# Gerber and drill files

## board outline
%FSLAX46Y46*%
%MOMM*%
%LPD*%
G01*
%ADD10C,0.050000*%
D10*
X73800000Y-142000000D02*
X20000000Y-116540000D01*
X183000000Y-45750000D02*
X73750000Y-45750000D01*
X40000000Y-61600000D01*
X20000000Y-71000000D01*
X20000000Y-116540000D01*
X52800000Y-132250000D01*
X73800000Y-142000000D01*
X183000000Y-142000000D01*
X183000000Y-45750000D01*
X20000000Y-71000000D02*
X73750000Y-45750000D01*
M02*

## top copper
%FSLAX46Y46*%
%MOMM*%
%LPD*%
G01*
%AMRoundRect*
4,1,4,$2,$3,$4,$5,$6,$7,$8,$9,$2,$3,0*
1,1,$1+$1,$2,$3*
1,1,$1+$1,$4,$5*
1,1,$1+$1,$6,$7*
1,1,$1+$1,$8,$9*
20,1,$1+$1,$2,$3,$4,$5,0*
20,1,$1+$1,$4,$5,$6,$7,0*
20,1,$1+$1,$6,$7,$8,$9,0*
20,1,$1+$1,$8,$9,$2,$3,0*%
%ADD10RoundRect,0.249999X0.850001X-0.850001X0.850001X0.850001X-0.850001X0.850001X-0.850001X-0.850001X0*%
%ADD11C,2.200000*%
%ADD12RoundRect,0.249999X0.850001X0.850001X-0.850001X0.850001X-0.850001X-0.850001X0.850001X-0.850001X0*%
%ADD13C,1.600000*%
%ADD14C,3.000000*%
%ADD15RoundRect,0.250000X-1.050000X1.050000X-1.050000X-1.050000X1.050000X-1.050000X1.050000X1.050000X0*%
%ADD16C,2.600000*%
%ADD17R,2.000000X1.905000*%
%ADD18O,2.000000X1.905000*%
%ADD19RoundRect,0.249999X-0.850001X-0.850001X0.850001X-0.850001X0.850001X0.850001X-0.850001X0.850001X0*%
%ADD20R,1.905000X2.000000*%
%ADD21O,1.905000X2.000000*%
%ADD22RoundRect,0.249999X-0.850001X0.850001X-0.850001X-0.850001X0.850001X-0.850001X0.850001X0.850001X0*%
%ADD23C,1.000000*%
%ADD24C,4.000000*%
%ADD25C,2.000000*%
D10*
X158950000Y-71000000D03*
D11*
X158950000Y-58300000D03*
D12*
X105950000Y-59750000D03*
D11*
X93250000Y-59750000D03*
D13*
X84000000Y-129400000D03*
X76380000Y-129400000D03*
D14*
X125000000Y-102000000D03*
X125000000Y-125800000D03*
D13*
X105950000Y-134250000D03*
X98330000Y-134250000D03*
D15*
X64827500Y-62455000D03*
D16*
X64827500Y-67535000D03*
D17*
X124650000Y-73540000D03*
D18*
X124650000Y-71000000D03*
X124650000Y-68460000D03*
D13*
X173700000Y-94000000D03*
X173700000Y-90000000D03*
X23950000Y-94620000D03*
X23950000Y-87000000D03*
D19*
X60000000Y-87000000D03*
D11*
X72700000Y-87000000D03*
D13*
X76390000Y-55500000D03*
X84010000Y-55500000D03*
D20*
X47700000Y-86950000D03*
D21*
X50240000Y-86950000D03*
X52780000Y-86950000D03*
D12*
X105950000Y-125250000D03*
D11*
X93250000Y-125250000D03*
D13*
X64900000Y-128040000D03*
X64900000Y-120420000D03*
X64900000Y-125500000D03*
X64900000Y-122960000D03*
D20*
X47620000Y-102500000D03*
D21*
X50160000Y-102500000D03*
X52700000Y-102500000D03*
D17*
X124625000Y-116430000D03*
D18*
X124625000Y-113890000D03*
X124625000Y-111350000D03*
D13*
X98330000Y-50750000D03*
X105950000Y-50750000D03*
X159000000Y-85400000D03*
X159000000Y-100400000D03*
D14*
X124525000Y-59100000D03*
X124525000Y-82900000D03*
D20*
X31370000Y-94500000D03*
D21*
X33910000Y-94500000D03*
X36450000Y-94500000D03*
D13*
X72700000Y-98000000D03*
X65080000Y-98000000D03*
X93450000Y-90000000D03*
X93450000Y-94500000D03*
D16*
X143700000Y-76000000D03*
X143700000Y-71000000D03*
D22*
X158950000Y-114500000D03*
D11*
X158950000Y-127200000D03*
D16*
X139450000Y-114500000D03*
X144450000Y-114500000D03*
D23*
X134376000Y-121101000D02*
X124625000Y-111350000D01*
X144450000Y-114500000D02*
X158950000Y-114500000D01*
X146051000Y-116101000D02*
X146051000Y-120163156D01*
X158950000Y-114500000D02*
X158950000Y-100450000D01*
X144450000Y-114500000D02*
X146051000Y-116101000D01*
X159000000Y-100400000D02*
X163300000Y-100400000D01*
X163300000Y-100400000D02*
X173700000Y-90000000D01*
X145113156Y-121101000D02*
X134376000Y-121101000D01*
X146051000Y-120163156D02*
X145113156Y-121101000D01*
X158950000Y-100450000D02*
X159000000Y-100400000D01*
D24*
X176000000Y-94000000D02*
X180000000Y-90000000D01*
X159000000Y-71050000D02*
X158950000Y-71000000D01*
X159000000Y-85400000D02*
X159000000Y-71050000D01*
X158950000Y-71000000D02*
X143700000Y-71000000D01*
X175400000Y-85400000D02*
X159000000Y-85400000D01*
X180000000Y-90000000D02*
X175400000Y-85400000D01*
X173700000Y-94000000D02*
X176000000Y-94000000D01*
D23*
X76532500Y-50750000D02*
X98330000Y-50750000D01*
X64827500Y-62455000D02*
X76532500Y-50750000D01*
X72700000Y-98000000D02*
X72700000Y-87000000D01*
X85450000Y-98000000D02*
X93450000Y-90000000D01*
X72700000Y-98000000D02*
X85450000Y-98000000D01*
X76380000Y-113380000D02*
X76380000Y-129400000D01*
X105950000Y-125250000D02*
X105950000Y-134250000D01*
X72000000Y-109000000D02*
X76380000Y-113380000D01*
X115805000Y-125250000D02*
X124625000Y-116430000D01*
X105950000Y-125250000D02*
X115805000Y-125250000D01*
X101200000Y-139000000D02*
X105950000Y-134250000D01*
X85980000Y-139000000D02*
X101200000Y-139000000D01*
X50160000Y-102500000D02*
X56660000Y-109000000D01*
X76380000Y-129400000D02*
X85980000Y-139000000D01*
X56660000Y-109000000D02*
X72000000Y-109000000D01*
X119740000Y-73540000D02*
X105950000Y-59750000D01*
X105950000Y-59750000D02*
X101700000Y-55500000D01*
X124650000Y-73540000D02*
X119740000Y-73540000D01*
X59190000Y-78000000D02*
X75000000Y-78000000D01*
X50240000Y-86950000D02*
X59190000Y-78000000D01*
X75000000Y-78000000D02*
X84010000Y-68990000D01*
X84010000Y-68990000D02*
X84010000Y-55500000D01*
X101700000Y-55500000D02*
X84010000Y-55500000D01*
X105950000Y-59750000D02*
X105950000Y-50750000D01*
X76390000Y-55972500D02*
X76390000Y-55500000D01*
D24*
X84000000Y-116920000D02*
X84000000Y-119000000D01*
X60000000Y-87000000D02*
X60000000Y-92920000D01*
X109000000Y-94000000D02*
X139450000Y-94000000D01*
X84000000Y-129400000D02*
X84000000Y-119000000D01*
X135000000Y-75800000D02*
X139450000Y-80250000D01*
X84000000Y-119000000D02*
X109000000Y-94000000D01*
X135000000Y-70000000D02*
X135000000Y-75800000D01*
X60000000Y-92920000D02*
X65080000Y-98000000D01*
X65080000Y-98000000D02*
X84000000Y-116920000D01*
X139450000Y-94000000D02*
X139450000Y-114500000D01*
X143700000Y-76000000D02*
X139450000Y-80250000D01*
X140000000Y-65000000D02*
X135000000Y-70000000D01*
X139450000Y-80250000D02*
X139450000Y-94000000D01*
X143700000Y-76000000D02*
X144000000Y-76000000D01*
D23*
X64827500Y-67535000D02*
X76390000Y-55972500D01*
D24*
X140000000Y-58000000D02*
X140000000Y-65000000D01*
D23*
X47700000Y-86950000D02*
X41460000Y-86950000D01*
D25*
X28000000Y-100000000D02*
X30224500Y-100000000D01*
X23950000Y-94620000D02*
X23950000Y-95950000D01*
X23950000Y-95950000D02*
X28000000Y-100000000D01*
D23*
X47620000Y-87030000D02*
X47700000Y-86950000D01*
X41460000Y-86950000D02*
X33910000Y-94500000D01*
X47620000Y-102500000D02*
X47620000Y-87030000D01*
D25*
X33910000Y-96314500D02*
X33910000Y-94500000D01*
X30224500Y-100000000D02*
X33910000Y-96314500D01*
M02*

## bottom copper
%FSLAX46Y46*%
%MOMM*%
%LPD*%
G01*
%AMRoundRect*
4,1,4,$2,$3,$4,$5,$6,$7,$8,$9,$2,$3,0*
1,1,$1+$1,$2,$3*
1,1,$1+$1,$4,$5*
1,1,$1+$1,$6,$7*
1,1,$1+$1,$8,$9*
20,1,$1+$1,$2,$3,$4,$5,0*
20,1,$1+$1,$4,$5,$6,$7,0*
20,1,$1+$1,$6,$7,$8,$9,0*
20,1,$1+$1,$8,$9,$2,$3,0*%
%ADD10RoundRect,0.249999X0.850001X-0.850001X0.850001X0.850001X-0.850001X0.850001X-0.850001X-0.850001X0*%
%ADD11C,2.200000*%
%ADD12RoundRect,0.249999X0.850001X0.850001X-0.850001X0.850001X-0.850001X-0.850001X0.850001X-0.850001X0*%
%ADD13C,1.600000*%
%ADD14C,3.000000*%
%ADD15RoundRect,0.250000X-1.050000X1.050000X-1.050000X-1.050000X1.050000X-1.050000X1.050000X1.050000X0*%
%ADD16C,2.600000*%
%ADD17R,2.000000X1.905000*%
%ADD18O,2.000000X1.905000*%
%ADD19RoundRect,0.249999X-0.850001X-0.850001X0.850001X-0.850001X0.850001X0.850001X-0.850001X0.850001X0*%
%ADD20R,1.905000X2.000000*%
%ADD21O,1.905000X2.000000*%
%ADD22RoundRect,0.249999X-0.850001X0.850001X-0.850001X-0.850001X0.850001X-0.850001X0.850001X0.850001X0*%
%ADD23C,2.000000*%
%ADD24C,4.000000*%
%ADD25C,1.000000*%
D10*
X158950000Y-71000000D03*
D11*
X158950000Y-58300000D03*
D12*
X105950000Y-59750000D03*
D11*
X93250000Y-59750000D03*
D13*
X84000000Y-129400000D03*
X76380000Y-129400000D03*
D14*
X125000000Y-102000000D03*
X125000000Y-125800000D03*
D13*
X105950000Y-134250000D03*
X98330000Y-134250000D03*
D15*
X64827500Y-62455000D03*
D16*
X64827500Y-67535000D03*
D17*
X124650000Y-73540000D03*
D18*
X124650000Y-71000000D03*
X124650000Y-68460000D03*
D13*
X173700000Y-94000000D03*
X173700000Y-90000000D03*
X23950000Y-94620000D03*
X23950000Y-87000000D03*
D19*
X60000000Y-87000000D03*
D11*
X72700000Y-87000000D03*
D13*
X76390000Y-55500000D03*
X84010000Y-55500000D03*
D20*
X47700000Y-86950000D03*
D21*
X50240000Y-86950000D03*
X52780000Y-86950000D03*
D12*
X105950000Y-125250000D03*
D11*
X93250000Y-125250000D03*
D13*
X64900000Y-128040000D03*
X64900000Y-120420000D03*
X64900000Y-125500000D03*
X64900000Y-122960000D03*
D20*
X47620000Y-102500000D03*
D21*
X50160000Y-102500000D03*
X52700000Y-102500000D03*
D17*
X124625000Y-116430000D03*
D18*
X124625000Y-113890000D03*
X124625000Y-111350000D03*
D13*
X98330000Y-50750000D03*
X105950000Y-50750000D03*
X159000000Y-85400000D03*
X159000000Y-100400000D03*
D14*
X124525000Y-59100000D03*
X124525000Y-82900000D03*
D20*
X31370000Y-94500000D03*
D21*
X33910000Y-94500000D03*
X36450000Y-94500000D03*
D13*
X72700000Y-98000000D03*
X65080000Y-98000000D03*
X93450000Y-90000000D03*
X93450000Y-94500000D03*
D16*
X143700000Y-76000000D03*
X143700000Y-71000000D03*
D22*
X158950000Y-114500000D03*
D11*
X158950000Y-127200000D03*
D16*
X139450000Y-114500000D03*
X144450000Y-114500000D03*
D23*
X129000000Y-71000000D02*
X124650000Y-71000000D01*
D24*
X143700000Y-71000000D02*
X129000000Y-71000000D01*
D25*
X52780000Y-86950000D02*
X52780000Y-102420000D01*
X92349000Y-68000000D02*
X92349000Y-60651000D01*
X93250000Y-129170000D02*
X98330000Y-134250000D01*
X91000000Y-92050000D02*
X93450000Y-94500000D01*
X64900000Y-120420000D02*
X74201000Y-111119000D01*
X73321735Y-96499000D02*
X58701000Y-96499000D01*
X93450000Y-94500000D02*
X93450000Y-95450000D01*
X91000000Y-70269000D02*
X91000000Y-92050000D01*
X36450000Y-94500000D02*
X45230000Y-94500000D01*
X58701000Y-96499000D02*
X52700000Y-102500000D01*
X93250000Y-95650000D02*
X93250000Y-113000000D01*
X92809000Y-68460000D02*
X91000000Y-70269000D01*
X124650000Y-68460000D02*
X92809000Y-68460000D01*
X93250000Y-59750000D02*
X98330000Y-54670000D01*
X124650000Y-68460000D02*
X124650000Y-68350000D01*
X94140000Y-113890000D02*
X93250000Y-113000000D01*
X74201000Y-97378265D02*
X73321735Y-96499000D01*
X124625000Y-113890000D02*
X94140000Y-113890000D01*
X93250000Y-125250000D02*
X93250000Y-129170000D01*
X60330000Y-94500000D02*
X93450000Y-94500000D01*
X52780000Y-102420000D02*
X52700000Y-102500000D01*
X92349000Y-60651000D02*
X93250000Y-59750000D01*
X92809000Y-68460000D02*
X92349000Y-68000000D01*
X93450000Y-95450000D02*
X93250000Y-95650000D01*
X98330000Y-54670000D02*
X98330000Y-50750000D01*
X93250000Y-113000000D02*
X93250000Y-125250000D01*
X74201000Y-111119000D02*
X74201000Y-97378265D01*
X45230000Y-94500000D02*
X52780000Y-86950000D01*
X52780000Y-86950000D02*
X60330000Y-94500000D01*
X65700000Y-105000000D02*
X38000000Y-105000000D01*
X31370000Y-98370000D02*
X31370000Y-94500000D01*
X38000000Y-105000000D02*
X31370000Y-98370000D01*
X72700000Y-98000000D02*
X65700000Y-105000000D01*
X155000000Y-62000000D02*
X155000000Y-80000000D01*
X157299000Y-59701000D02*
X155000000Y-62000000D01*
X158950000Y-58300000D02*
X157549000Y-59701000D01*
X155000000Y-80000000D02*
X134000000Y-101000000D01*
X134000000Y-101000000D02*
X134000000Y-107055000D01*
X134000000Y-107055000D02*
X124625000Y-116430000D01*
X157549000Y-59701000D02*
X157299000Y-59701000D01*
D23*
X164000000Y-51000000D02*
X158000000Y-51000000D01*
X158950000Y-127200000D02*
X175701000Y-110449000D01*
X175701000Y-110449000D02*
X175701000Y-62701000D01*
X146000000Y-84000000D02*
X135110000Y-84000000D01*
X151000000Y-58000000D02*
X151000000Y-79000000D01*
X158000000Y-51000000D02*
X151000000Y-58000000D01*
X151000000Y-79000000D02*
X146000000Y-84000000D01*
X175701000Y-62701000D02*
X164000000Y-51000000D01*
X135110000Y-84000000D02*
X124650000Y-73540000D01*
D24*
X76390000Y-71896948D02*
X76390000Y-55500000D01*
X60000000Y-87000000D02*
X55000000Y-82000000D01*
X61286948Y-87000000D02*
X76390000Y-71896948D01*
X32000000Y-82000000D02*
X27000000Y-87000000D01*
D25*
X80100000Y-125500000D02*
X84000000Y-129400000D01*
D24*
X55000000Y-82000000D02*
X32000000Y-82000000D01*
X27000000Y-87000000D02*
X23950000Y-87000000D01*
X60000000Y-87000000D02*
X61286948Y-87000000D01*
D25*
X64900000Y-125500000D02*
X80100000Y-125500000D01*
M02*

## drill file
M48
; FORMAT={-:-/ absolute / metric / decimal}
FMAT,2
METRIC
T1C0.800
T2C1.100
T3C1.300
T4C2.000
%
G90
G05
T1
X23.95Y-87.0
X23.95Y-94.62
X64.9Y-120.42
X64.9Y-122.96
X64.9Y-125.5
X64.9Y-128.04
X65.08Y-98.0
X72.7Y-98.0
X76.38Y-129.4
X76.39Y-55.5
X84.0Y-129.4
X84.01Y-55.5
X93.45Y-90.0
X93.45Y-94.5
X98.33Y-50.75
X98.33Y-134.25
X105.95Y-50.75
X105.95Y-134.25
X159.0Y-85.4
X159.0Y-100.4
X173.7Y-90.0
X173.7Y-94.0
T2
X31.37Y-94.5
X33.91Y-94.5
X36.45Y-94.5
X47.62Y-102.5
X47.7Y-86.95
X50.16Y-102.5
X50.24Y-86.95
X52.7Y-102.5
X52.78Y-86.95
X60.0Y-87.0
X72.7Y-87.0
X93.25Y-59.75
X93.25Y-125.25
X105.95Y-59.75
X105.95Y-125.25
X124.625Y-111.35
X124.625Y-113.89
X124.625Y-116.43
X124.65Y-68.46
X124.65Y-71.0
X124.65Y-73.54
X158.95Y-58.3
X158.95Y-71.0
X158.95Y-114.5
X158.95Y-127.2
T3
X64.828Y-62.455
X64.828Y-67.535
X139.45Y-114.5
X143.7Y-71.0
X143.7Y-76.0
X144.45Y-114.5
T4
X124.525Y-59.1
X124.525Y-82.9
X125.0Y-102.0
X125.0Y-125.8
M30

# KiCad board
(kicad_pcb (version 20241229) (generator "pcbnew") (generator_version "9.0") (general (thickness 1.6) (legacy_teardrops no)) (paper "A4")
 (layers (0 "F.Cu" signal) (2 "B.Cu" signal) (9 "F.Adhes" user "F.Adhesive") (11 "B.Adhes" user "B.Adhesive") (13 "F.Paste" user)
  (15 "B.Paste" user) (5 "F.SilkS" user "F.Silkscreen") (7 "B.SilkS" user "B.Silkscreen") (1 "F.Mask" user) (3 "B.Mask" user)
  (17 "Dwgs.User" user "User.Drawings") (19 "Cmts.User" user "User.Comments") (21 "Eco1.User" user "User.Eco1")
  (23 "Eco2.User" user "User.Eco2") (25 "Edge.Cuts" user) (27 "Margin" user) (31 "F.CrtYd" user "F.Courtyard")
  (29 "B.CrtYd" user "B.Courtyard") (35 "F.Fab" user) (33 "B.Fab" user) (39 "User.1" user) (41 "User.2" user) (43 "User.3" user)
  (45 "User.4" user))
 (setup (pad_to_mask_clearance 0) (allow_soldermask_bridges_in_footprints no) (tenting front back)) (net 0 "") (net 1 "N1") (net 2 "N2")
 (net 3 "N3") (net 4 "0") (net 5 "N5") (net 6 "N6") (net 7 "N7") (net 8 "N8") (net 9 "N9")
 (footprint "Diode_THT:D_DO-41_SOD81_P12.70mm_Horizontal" (layer "F.Cu") (at 158.95 71 90)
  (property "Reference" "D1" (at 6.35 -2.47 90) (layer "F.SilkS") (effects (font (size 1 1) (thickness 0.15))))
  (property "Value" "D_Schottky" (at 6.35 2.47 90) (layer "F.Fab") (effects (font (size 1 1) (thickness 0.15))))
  (pad "1" thru_hole roundrect (at 0 0 90) (size 2.2 2.2) (drill 1.1) (layers "*.Cu" "*.Mask") (remove_unused_layers no)
   (roundrect_rratio 0.113636) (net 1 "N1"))
  (pad "2" thru_hole circle (at 12.7 0 90) (size 2.2 2.2) (drill 1.1) (layers "*.Cu" "*.Mask") (remove_unused_layers no) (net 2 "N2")))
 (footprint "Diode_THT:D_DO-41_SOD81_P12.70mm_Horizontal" (layer "F.Cu") (at 105.95 59.75 180)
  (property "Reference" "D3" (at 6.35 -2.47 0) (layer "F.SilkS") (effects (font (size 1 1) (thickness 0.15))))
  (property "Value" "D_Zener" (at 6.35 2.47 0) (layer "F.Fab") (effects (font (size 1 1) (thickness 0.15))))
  (pad "1" thru_hole roundrect (at 0 0 180) (size 2.2 2.2) (drill 1.1) (layers "*.Cu" "*.Mask") (remove_unused_layers no)
   (roundrect_rratio 0.113636) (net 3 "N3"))
  (pad "2" thru_hole circle (at 12.7 0 180) (size 2.2 2.2) (drill 1.1) (layers "*.Cu" "*.Mask") (remove_unused_layers no) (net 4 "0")))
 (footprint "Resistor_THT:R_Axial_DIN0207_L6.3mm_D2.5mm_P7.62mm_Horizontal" (layer "F.Cu") (at 84 129.4 180)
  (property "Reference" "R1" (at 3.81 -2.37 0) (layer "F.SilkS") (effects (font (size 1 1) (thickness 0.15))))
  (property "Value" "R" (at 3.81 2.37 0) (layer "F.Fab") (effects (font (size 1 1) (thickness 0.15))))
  (pad "1" thru_hole circle (at 0 0 180) (size 1.6 1.6) (drill 0.8) (layers "*.Cu" "*.Mask") (remove_unused_layers no) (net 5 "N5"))
  (pad "2" thru_hole circle (at 7.62 0 180) (size 1.6 1.6) (drill 0.8) (layers "*.Cu" "*.Mask") (remove_unused_layers no) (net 2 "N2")))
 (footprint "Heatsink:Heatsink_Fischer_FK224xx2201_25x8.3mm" (layer "F.Cu") (at 125 102 -90)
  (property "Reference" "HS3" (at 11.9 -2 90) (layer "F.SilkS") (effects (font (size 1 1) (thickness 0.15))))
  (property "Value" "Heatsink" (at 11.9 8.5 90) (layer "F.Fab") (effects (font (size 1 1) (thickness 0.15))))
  (pad "1" thru_hole circle (at 0 0 270) (size 3 3) (drill 2) (layers "*.Cu" "*.Mask") (remove_unused_layers no))
  (pad "1" thru_hole circle (at 23.8 0 270) (size 3 3) (drill 2) (layers "*.Cu" "*.Mask") (remove_unused_layers no)))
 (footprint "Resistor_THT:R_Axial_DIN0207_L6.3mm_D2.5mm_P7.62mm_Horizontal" (layer "F.Cu") (at 105.95 134.25 180)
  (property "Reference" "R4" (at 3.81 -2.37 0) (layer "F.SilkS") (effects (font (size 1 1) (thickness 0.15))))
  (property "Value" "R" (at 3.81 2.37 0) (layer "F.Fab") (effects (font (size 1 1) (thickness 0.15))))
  (pad "1" thru_hole circle (at 0 0 180) (size 1.6 1.6) (drill 0.8) (layers "*.Cu" "*.Mask") (remove_unused_layers no) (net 2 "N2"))
  (pad "2" thru_hole circle (at 7.62 0 180) (size 1.6 1.6) (drill 0.8) (layers "*.Cu" "*.Mask") (remove_unused_layers no) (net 4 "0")))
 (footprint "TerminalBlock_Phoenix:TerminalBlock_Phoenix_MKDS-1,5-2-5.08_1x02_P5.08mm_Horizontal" (layer "F.Cu") (at 64.8275 62.455 -90)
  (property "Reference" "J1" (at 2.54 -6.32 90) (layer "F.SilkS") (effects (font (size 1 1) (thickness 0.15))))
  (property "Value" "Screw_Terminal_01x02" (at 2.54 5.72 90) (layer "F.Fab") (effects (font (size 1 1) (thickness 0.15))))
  (pad "1" thru_hole roundrect (at 0 0 270) (size 2.6 2.6) (drill 1.3) (layers "*.Cu" "*.Mask") (remove_unused_layers no)
   (roundrect_rratio 0.096154) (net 4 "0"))
  (pad "2" thru_hole circle (at 5.08 0 270) (size 2.6 2.6) (drill 1.3) (layers "*.Cu" "*.Mask") (remove_unused_layers no) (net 5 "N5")))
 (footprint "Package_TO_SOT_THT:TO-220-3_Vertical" (layer "F.Cu") (at 124.65 73.54 90)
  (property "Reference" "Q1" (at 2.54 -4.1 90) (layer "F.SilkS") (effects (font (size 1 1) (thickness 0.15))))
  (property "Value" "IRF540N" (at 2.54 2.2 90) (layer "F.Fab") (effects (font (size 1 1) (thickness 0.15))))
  (pad "1" thru_hole rect (at 0 0 90) (size 1.905 2) (drill 1.1) (layers "*.Cu" "*.Mask") (remove_unused_layers no) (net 3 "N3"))
  (pad "2" thru_hole oval (at 2.54 0 90) (size 1.905 2) (drill 1.1) (layers "*.Cu" "*.Mask") (remove_unused_layers no) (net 1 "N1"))
  (pad "3" thru_hole oval (at 5.08 0 90) (size 1.905 2) (drill 1.1) (layers "*.Cu" "*.Mask") (remove_unused_layers no) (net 4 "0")))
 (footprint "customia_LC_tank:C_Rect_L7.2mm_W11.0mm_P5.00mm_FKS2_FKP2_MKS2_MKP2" (layer "F.Cu") (at 248.7 94.5 180)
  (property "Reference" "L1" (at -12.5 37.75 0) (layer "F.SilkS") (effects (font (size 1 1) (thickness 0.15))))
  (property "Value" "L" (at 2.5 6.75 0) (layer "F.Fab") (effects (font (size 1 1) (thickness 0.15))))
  (pad "1" thru_hole circle (at 75 0.5 180) (size 1.6 1.6) (drill 0.8) (layers "*.Cu" "*.Mask") (remove_unused_layers no) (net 1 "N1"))
  (pad "2" thru_hole circle (at 75 4.5 180) (size 1.6 1.6) (drill 0.8) (layers "*.Cu" "*.Mask") (remove_unused_layers no) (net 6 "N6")))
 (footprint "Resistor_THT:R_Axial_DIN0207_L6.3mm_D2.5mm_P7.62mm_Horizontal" (layer "F.Cu") (at 23.95 94.62 90)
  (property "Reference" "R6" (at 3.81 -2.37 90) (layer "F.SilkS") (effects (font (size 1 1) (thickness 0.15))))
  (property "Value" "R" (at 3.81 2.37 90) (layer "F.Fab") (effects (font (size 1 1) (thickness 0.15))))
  (pad "1" thru_hole circle (at 0 0 90) (size 1.6 1.6) (drill 0.8) (layers "*.Cu" "*.Mask") (remove_unused_layers no) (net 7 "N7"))
  (pad "2" thru_hole circle (at 7.62 0 90) (size 1.6 1.6) (drill 0.8) (layers "*.Cu" "*.Mask") (remove_unused_layers no) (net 5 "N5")))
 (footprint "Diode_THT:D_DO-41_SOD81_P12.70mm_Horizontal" (layer "F.Cu") (at 60 87)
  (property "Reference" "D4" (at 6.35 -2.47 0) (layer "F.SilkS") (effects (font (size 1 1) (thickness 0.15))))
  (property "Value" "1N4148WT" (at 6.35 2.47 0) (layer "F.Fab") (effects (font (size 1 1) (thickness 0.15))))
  (pad "1" thru_hole roundrect (at 0 0) (size 2.2 2.2) (drill 1.1) (layers "*.Cu" "*.Mask") (remove_unused_layers no)
   (roundrect_rratio 0.113636) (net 5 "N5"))
  (pad "2" thru_hole circle (at 12.7 0) (size 2.2 2.2) (drill 1.1) (layers "*.Cu" "*.Mask") (remove_unused_layers no) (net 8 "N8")))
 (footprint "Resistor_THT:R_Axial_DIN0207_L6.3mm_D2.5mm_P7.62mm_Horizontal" (layer "F.Cu") (at 76.39 55.5)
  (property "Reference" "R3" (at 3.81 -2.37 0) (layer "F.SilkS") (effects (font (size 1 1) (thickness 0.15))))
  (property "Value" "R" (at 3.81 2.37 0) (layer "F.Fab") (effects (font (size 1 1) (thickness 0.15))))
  (pad "1" thru_hole circle (at 0 0) (size 1.6 1.6) (drill 0.8) (layers "*.Cu" "*.Mask") (remove_unused_layers no) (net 5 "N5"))
  (pad "2" thru_hole circle (at 7.62 0) (size 1.6 1.6) (drill 0.8) (layers "*.Cu" "*.Mask") (remove_unused_layers no) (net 3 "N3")))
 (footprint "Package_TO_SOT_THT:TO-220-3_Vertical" (layer "F.Cu") (at 47.7 86.95)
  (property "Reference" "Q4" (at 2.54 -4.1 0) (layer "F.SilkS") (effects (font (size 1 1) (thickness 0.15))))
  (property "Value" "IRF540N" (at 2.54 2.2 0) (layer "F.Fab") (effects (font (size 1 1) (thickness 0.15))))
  (pad "1" thru_hole rect (at 0 0) (size 1.905 2) (drill 1.1) (layers "*.Cu" "*.Mask") (remove_unused_layers no) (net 7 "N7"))
  (pad "2" thru_hole oval (at 2.54 0) (size 1.905 2) (drill 1.1) (layers "*.Cu" "*.Mask") (remove_unused_layers no) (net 3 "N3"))
  (pad "3" thru_hole oval (at 5.08 0) (size 1.905 2) (drill 1.1) (layers "*.Cu" "*.Mask") (remove_unused_layers no) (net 4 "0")))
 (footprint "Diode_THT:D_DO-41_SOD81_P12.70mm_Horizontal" (layer "F.Cu") (at 105.95 125.25 180)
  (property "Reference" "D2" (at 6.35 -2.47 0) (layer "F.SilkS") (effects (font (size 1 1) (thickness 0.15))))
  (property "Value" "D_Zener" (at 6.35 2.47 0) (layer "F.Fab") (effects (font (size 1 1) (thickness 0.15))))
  (pad "1" thru_hole roundrect (at 0 0 180) (size 2.2 2.2) (drill 1.1) (layers "*.Cu" "*.Mask") (remove_unused_layers no)
   (roundrect_rratio 0.113636) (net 2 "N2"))
  (pad "2" thru_hole circle (at 12.7 0 180) (size 2.2 2.2) (drill 1.1) (layers "*.Cu" "*.Mask") (remove_unused_layers no) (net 4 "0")))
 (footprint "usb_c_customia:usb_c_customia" (layer "F.Cu") (at 64.9 128.04 90)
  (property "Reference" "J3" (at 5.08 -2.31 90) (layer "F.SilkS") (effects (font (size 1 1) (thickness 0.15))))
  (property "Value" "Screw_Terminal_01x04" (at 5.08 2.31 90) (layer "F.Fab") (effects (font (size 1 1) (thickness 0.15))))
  (pad "2" thru_hole circle (at 0 0 90) (size 1.6 1.6) (drill 0.8) (layers "*.Cu" "*.Mask") (remove_unused_layers no) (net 4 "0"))
  (pad "2" thru_hole circle (at 7.62 0 90) (size 1.6 1.6) (drill 0.8) (layers "*.Cu" "*.Mask") (remove_unused_layers no) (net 4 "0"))
  (pad "3" thru_hole circle (at 2.54 0 90) (size 1.6 1.6) (drill 0.8) (layers "*.Cu" "*.Mask") (remove_unused_layers no) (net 5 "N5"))
  (pad "4" thru_hole circle (at 5.08 0 90) (size 1.6 1.6) (drill 0.8) (layers "*.Cu" "*.Mask") (remove_unused_layers no) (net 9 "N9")))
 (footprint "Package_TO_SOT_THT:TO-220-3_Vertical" (layer "F.Cu") (at 47.62 102.5)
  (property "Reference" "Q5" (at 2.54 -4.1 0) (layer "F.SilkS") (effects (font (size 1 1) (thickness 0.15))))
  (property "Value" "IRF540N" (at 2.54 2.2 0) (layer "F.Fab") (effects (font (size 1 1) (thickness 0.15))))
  (pad "1" thru_hole rect (at 0 0) (size 1.905 2) (drill 1.1) (layers "*.Cu" "*.Mask") (remove_unused_layers no) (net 7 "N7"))
  (pad "2" thru_hole oval (at 2.54 0) (size 1.905 2) (drill 1.1) (layers "*.Cu" "*.Mask") (remove_unused_layers no) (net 2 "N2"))
  (pad "3" thru_hole oval (at 5.08 0) (size 1.905 2) (drill 1.1) (layers "*.Cu" "*.Mask") (remove_unused_layers no) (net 4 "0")))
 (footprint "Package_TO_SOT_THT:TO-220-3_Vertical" (layer "F.Cu") (at 124.625 116.43 90)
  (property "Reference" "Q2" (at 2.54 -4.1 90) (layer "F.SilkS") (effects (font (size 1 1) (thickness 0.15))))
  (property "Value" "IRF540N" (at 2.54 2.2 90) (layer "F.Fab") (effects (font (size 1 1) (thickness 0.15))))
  (pad "1" thru_hole rect (at 0 0 90) (size 1.905 2) (drill 1.1) (layers "*.Cu" "*.Mask") (remove_unused_layers no) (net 2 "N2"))
  (pad "2" thru_hole oval (at 2.54 0 90) (size 1.905 2) (drill 1.1) (layers "*.Cu" "*.Mask") (remove_unused_layers no) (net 4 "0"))
  (pad "3" thru_hole oval (at 5.08 0 90) (size 1.905 2) (drill 1.1) (layers "*.Cu" "*.Mask") (remove_unused_layers no) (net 6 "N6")))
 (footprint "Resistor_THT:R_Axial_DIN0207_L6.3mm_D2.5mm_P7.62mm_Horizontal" (layer "F.Cu") (at 98.33 50.75)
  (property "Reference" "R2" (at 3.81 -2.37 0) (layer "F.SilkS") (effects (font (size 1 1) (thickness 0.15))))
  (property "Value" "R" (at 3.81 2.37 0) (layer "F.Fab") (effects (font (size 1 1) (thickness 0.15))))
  (pad "1" thru_hole circle (at 0 0) (size 1.6 1.6) (drill 0.8) (layers "*.Cu" "*.Mask") (remove_unused_layers no) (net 4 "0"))
  (pad "2" thru_hole circle (at 7.62 0) (size 1.6 1.6) (drill 0.8) (layers "*.Cu" "*.Mask") (remove_unused_layers no) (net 3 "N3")))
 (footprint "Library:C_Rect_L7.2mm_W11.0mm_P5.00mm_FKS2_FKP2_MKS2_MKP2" (layer "F.Cu") (at 159.1 93.1 -90)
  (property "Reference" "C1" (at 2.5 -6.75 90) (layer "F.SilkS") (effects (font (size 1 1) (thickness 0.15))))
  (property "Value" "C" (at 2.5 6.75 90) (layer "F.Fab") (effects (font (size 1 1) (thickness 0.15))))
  (pad "1" thru_hole circle (at -7.7 0.1 270) (size 1.6 1.6) (drill 0.8) (layers "*.Cu" "*.Mask") (remove_unused_layers no) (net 1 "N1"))
  (pad "2" thru_hole circle (at 7.3 0.1 270) (size 1.6 1.6) (drill 0.8) (layers "*.Cu" "*.Mask") (remove_unused_layers no) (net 6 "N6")))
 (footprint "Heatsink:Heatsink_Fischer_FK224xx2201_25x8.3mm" (layer "F.Cu") (at 124.525 59.1 -90)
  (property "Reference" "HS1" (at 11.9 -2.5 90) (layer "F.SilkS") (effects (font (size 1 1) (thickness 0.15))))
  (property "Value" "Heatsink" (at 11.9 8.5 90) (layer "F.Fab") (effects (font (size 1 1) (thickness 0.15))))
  (pad "1" thru_hole circle (at 0 0 270) (size 3 3) (drill 2) (layers "*.Cu" "*.Mask") (remove_unused_layers no))
  (pad "1" thru_hole circle (at 23.8 0 270) (size 3 3) (drill 2) (layers "*.Cu" "*.Mask") (remove_unused_layers no)))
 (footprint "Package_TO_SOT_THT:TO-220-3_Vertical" (layer "F.Cu") (at 31.37 94.5)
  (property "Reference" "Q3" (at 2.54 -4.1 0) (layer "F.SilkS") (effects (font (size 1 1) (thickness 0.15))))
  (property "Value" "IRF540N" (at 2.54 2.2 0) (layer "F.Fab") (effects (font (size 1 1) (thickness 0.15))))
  (pad "1" thru_hole rect (at 0 0) (size 1.905 2) (drill 1.1) (layers "*.Cu" "*.Mask") (remove_unused_layers no) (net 8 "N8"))
  (pad "2" thru_hole oval (at 2.54 0) (size 1.905 2) (drill 1.1) (layers "*.Cu" "*.Mask") (remove_unused_layers no) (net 7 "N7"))
  (pad "3" thru_hole oval (at 5.08 0) (size 1.905 2) (drill 1.1) (layers "*.Cu" "*.Mask") (remove_unused_layers no) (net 4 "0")))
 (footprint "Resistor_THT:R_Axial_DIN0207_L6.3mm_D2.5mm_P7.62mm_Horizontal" (layer "F.Cu") (at 72.7 98 180)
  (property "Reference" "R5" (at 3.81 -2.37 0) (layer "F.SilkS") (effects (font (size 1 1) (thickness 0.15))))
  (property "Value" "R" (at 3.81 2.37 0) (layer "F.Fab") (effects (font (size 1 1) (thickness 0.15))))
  (pad "1" thru_hole circle (at 0 0 180) (size 1.6 1.6) (drill 0.8) (layers "*.Cu" "*.Mask") (remove_unused_layers no) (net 8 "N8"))
  (pad "2" thru_hole circle (at 7.62 0 180) (size 1.6 1.6) (drill 0.8) (layers "*.Cu" "*.Mask") (remove_unused_layers no) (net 5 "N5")))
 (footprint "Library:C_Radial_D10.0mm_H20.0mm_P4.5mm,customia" (layer "F.Cu") (at 93.45 89.75 -90)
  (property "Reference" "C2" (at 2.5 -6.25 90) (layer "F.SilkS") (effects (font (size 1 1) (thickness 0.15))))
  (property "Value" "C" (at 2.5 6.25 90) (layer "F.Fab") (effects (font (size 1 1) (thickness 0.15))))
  (pad "1" thru_hole circle (at 0.25 0 270) (size 1.6 1.6) (drill 0.8) (layers "*.Cu" "*.Mask") (remove_unused_layers no) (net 8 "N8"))
  (pad "2" thru_hole circle (at 4.75 0 270) (size 1.6 1.6) (drill 0.8) (layers "*.Cu" "*.Mask") (remove_unused_layers no) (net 4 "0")))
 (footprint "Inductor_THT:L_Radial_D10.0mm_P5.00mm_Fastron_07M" (layer "F.Cu") (at 143.7 76 90)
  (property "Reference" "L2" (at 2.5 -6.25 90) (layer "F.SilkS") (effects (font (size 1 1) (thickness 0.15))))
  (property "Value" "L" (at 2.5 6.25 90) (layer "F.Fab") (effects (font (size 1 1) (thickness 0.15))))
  (pad "1" thru_hole circle (at 0 0 90) (size 2.6 2.6) (drill 1.3) (layers "*.Cu" "*.Mask") (remove_unused_layers no) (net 5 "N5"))
  (pad "2" thru_hole circle (at 5 0 90) (size 2.6 2.6) (drill 1.3) (layers "*.Cu" "*.Mask") (remove_unused_layers no) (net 1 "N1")))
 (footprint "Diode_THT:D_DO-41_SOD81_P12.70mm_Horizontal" (layer "F.Cu") (at 158.95 114.5 -90)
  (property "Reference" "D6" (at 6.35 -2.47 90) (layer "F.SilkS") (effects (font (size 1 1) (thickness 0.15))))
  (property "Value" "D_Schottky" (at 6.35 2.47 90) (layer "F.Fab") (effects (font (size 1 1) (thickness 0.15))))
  (pad "1" thru_hole roundrect (at 0 0 270) (size 2.2 2.2) (drill 1.1) (layers "*.Cu" "*.Mask") (remove_unused_layers no)
   (roundrect_rratio 0.113636) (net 6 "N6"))
  (pad "2" thru_hole circle (at 12.7 0 270) (size 2.2 2.2) (drill 1.1) (layers "*.Cu" "*.Mask") (remove_unused_layers no) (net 3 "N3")))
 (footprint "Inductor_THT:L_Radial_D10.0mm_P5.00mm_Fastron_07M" (layer "F.Cu") (at 139.45 114.5)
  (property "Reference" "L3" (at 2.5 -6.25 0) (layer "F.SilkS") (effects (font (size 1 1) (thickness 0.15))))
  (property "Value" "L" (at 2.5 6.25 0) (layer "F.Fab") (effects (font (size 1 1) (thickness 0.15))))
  (pad "1" thru_hole circle (at 0 0) (size 2.6 2.6) (drill 1.3) (layers "*.Cu" "*.Mask") (remove_unused_layers no) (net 5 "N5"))
  (pad "2" thru_hole circle (at 5 0) (size 2.6 2.6) (drill 1.3) (layers "*.Cu" "*.Mask") (remove_unused_layers no) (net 6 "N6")))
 (gr_line (start 73.8 142) (end 20 116.54) (stroke (width 0.05) (type default)) (layer "Edge.Cuts"))
 (gr_poly
  (pts (xy 183 45.75) (xy 73.75 45.75) (xy 40 61.6) (xy 20 71) (xy 20 116.54) (xy 52.8 132.25) (xy 73.8 142) (xy 183 142))
  (stroke (width 0.05) (type solid)) (fill no) (layer "Edge.Cuts"))
 (gr_line (start 20 71) (end 73.75 45.75) (stroke (width 0.05) (type default)) (layer "Edge.Cuts"))
 (segment (start 134.376 121.101) (end 124.625 111.35) (width 1) (layer "F.Cu") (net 6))
 (segment (start 144.45 114.5) (end 158.95 114.5) (width 1) (layer "F.Cu") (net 6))
 (segment (start 146.051 116.101) (end 146.051 120.163156) (width 1) (layer "F.Cu") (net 6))
 (segment (start 158.95 114.5) (end 158.95 100.45) (width 1) (layer "F.Cu") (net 6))
 (segment (start 144.45 114.5) (end 146.051 116.101) (width 1) (layer "F.Cu") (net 6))
 (segment (start 159 100.4) (end 163.3 100.4) (width 1) (layer "F.Cu") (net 6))
 (segment (start 163.3 100.4) (end 173.7 90) (width 1) (layer "F.Cu") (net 6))
 (segment (start 145.113156 121.101) (end 134.376 121.101) (width 1) (layer "F.Cu") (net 6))
 (segment (start 146.051 120.163156) (end 145.113156 121.101) (width 1) (layer "F.Cu") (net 6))
 (segment (start 158.95 100.45) (end 159 100.4) (width 1) (layer "F.Cu") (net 6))
 (segment (start 176 94) (end 180 90) (width 4) (layer "F.Cu") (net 1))
 (segment (start 159 71.05) (end 158.95 71) (width 4) (layer "F.Cu") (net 1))
 (segment (start 159 85.4) (end 159 71.05) (width 4) (layer "F.Cu") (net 1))
 (segment (start 158.95 71) (end 143.7 71) (width 4) (layer "F.Cu") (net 1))
 (segment (start 175.4 85.4) (end 159 85.4) (width 4) (layer "F.Cu") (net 1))
 (segment (start 180 90) (end 175.4 85.4) (width 4) (layer "F.Cu") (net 1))
 (segment (start 173.7 94) (end 176 94) (width 4) (layer "F.Cu") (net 1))
 (segment (start 129 71) (end 124.65 71) (width 2) (layer "B.Cu") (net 1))
 (segment (start 143.7 71) (end 129 71) (width 4) (layer "B.Cu") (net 1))
 (segment (start 76.5325 50.75) (end 98.33 50.75) (width 1) (layer "F.Cu") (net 4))
 (segment (start 64.8275 62.455) (end 76.5325 50.75) (width 1) (layer "F.Cu") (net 4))
 (segment (start 52.78 86.95) (end 52.78 102.42) (width 1) (layer "B.Cu") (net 4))
 (segment (start 92.349 68) (end 92.349 60.651) (width 1) (layer "B.Cu") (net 4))
 (segment (start 93.25 129.17) (end 98.33 134.25) (width 1) (layer "B.Cu") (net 4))
 (segment (start 91 92.05) (end 93.45 94.5) (width 1) (layer "B.Cu") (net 4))
 (segment (start 64.9 120.42) (end 74.201 111.119) (width 1) (layer "B.Cu") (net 4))
 (segment (start 73.321735 96.499) (end 58.701 96.499) (width 1) (layer "B.Cu") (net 4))
 (segment (start 93.45 94.5) (end 93.45 95.45) (width 1) (layer "B.Cu") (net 4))
 (segment (start 91 70.269) (end 91 92.05) (width 1) (layer "B.Cu") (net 4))
 (segment (start 36.45 94.5) (end 45.23 94.5) (width 1) (layer "B.Cu") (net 4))
 (segment (start 58.701 96.499) (end 52.7 102.5) (width 1) (layer "B.Cu") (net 4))
 (segment (start 93.25 95.65) (end 93.25 113) (width 1) (layer "B.Cu") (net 4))
 (segment (start 92.809 68.46) (end 91 70.269) (width 1) (layer "B.Cu") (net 4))
 (segment (start 124.65 68.46) (end 92.809 68.46) (width 1) (layer "B.Cu") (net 4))
 (segment (start 93.25 59.75) (end 98.33 54.67) (width 1) (layer "B.Cu") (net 4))
 (segment (start 124.65 68.46) (end 124.65 68.35) (width 1) (layer "B.Cu") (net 4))
 (segment (start 94.14 113.89) (end 93.25 113) (width 1) (layer "B.Cu") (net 4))
 (segment (start 74.201 97.378265) (end 73.321735 96.499) (width 1) (layer "B.Cu") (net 4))
 (segment (start 124.625 113.89) (end 94.14 113.89) (width 1) (layer "B.Cu") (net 4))
 (segment (start 93.25 125.25) (end 93.25 129.17) (width 1) (layer "B.Cu") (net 4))
 (segment (start 60.33 94.5) (end 93.45 94.5) (width 1) (layer "B.Cu") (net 4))
 (segment (start 52.78 102.42) (end 52.7 102.5) (width 1) (layer "B.Cu") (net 4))
 (segment (start 92.349 60.651) (end 93.25 59.75) (width 1) (layer "B.Cu") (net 4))
 (segment (start 92.809 68.46) (end 92.349 68) (width 1) (layer "B.Cu") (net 4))
 (segment (start 93.45 95.45) (end 93.25 95.65) (width 1) (layer "B.Cu") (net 4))
 (segment (start 98.33 54.67) (end 98.33 50.75) (width 1) (layer "B.Cu") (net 4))
 (segment (start 93.25 113) (end 93.25 125.25) (width 1) (layer "B.Cu") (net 4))
 (segment (start 74.201 111.119) (end 74.201 97.378265) (width 1) (layer "B.Cu") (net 4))
 (segment (start 45.23 94.5) (end 52.78 86.95) (width 1) (layer "B.Cu") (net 4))
 (segment (start 52.78 86.95) (end 60.33 94.5) (width 1) (layer "B.Cu") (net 4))
 (segment (start 72.7 98) (end 72.7 87) (width 1) (layer "F.Cu") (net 8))
 (segment (start 85.45 98) (end 93.45 90) (width 1) (layer "F.Cu") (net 8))
 (segment (start 72.7 98) (end 85.45 98) (width 1) (layer "F.Cu") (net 8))
 (segment (start 65.7 105) (end 38 105) (width 1) (layer "B.Cu") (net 8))
 (segment (start 31.37 98.37) (end 31.37 94.5) (width 1) (layer "B.Cu") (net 8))
 (segment (start 38 105) (end 31.37 98.37) (width 1) (layer "B.Cu") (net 8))
 (segment (start 72.7 98) (end 65.7 105) (width 1) (layer "B.Cu") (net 8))
 (segment (start 76.38 113.38) (end 76.38 129.4) (width 1) (layer "F.Cu") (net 2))
 (segment (start 105.95 125.25) (end 105.95 134.25) (width 1) (layer "F.Cu") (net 2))
 (segment (start 72 109) (end 76.38 113.38) (width 1) (layer "F.Cu") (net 2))
 (segment (start 115.805 125.25) (end 124.625 116.43) (width 1) (layer "F.Cu") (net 2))
 (segment (start 105.95 125.25) (end 115.805 125.25) (width 1) (layer "F.Cu") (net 2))
 (segment (start 101.2 139) (end 105.95 134.25) (width 1) (layer "F.Cu") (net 2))
 (segment (start 85.98 139) (end 101.2 139) (width 1) (layer "F.Cu") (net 2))
 (segment (start 50.16 102.5) (end 56.66 109) (width 1) (layer "F.Cu") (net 2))
 (segment (start 76.38 129.4) (end 85.98 139) (width 1) (layer "F.Cu") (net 2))
 (segment (start 56.66 109) (end 72 109) (width 1) (layer "F.Cu") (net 2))
 (segment (start 155 62) (end 155 80) (width 1) (layer "B.Cu") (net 2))
 (segment (start 157.299 59.701) (end 155 62) (width 1) (layer "B.Cu") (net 2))
 (segment (start 158.95 58.3) (end 157.549 59.701) (width 1) (layer "B.Cu") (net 2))
 (segment (start 155 80) (end 134 101) (width 1) (layer "B.Cu") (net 2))
 (segment (start 134 101) (end 134 107.055) (width 1) (layer "B.Cu") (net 2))
 (segment (start 134 107.055) (end 124.625 116.43) (width 1) (layer "B.Cu") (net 2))
 (segment (start 157.549 59.701) (end 157.299 59.701) (width 1) (layer "B.Cu") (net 2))
 (segment (start 119.74 73.54) (end 105.95 59.75) (width 1) (layer "F.Cu") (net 3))
 (segment (start 105.95 59.75) (end 101.7 55.5) (width 1) (layer "F.Cu") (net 3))
 (segment (start 124.65 73.54) (end 119.74 73.54) (width 1) (layer "F.Cu") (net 3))
 (segment (start 59.19 78) (end 75 78) (width 1) (layer "F.Cu") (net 3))
 (segment (start 50.24 86.95) (end 59.19 78) (width 1) (layer "F.Cu") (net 3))
 (segment (start 75 78) (end 84.01 68.99) (width 1) (layer "F.Cu") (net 3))
 (segment (start 84.01 68.99) (end 84.01 55.5) (width 1) (layer "F.Cu") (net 3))
 (segment (start 101.7 55.5) (end 84.01 55.5) (width 1) (layer "F.Cu") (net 3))
 (segment (start 105.95 59.75) (end 105.95 50.75) (width 1) (layer "F.Cu") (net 3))
 (segment (start 164 51) (end 158 51) (width 2) (layer "B.Cu") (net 3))
 (segment (start 158.95 127.2) (end 175.701 110.449) (width 2) (layer "B.Cu") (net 3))
 (segment (start 175.701 110.449) (end 175.701 62.701) (width 2) (layer "B.Cu") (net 3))
 (segment (start 146 84) (end 135.11 84) (width 2) (layer "B.Cu") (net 3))
 (segment (start 151 58) (end 151 79) (width 2) (layer "B.Cu") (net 3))
 (segment (start 158 51) (end 151 58) (width 2) (layer "B.Cu") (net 3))
 (segment (start 151 79) (end 146 84) (width 2) (layer "B.Cu") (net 3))
 (segment (start 175.701 62.701) (end 164 51) (width 2) (layer "B.Cu") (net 3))
 (segment (start 135.11 84) (end 124.65 73.54) (width 2) (layer "B.Cu") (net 3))
 (segment (start 76.39 55.9725) (end 76.39 55.5) (width 1) (layer "F.Cu") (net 5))
 (segment (start 84 116.92) (end 84 119) (width 4) (layer "F.Cu") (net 5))
 (segment (start 60 87) (end 60 92.92) (width 4) (layer "F.Cu") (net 5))
 (segment (start 109 94) (end 139.45 94) (width 4) (layer "F.Cu") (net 5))
 (segment (start 84 129.4) (end 84 119) (width 4) (layer "F.Cu") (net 5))
 (segment (start 135 75.8) (end 139.45 80.25) (width 4) (layer "F.Cu") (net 5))
 (segment (start 84 119) (end 109 94) (width 4) (layer "F.Cu") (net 5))
 (segment (start 135 70) (end 135 75.8) (width 4) (layer "F.Cu") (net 5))
 (segment (start 60 92.92) (end 65.08 98) (width 4) (layer "F.Cu") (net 5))
 (segment (start 65.08 98) (end 84 116.92) (width 4) (layer "F.Cu") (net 5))
 (segment (start 139.45 94) (end 139.45 114.5) (width 4) (layer "F.Cu") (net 5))
 (segment (start 143.7 76) (end 139.45 80.25) (width 4) (layer "F.Cu") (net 5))
 (segment (start 140 65) (end 135 70) (width 4) (layer "F.Cu") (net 5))
 (segment (start 139.45 80.25) (end 139.45 94) (width 4) (layer "F.Cu") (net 5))
 (segment (start 143.7 76) (end 144 76) (width 4) (layer "F.Cu") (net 5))
 (segment (start 64.8275 67.535) (end 76.39 55.9725) (width 1) (layer "F.Cu") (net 5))
 (segment (start 140 58) (end 140 65) (width 4) (layer "F.Cu") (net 5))
 (segment (start 76.39 71.896948) (end 76.39 55.5) (width 4) (layer "B.Cu") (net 5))
 (segment (start 60 87) (end 55 82) (width 4) (layer "B.Cu") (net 5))
 (segment (start 61.286948 87) (end 76.39 71.896948) (width 4) (layer "B.Cu") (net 5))
 (segment (start 32 82) (end 27 87) (width 4) (layer "B.Cu") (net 5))
 (segment (start 80.1 125.5) (end 84 129.4) (width 1) (layer "B.Cu") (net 5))
 (segment (start 55 82) (end 32 82) (width 4) (layer "B.Cu") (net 5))
 (segment (start 27 87) (end 23.95 87) (width 4) (layer "B.Cu") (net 5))
 (segment (start 60 87) (end 61.286948 87) (width 4) (layer "B.Cu") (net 5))
 (segment (start 64.9 125.5) (end 80.1 125.5) (width 1) (layer "B.Cu") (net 5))
 (segment (start 47.7 86.95) (end 41.46 86.95) (width 1) (layer "F.Cu") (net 7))
 (segment (start 28 100) (end 30.2245 100) (width 2) (layer "F.Cu") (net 7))
 (segment (start 23.95 94.62) (end 23.95 95.95) (width 2) (layer "F.Cu") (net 7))
 (segment (start 23.95 95.95) (end 28 100) (width 2) (layer "F.Cu") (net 7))
 (segment (start 47.62 87.03) (end 47.7 86.95) (width 1) (layer "F.Cu") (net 7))
 (segment (start 41.46 86.95) (end 33.91 94.5) (width 1) (layer "F.Cu") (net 7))
 (segment (start 47.62 102.5) (end 47.62 87.03) (width 1) (layer "F.Cu") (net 7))
 (segment (start 33.91 96.3145) (end 33.91 94.5) (width 2) (layer "F.Cu") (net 7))
 (segment (start 30.2245 100) (end 33.91 96.3145) (width 2) (layer "F.Cu") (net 7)))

